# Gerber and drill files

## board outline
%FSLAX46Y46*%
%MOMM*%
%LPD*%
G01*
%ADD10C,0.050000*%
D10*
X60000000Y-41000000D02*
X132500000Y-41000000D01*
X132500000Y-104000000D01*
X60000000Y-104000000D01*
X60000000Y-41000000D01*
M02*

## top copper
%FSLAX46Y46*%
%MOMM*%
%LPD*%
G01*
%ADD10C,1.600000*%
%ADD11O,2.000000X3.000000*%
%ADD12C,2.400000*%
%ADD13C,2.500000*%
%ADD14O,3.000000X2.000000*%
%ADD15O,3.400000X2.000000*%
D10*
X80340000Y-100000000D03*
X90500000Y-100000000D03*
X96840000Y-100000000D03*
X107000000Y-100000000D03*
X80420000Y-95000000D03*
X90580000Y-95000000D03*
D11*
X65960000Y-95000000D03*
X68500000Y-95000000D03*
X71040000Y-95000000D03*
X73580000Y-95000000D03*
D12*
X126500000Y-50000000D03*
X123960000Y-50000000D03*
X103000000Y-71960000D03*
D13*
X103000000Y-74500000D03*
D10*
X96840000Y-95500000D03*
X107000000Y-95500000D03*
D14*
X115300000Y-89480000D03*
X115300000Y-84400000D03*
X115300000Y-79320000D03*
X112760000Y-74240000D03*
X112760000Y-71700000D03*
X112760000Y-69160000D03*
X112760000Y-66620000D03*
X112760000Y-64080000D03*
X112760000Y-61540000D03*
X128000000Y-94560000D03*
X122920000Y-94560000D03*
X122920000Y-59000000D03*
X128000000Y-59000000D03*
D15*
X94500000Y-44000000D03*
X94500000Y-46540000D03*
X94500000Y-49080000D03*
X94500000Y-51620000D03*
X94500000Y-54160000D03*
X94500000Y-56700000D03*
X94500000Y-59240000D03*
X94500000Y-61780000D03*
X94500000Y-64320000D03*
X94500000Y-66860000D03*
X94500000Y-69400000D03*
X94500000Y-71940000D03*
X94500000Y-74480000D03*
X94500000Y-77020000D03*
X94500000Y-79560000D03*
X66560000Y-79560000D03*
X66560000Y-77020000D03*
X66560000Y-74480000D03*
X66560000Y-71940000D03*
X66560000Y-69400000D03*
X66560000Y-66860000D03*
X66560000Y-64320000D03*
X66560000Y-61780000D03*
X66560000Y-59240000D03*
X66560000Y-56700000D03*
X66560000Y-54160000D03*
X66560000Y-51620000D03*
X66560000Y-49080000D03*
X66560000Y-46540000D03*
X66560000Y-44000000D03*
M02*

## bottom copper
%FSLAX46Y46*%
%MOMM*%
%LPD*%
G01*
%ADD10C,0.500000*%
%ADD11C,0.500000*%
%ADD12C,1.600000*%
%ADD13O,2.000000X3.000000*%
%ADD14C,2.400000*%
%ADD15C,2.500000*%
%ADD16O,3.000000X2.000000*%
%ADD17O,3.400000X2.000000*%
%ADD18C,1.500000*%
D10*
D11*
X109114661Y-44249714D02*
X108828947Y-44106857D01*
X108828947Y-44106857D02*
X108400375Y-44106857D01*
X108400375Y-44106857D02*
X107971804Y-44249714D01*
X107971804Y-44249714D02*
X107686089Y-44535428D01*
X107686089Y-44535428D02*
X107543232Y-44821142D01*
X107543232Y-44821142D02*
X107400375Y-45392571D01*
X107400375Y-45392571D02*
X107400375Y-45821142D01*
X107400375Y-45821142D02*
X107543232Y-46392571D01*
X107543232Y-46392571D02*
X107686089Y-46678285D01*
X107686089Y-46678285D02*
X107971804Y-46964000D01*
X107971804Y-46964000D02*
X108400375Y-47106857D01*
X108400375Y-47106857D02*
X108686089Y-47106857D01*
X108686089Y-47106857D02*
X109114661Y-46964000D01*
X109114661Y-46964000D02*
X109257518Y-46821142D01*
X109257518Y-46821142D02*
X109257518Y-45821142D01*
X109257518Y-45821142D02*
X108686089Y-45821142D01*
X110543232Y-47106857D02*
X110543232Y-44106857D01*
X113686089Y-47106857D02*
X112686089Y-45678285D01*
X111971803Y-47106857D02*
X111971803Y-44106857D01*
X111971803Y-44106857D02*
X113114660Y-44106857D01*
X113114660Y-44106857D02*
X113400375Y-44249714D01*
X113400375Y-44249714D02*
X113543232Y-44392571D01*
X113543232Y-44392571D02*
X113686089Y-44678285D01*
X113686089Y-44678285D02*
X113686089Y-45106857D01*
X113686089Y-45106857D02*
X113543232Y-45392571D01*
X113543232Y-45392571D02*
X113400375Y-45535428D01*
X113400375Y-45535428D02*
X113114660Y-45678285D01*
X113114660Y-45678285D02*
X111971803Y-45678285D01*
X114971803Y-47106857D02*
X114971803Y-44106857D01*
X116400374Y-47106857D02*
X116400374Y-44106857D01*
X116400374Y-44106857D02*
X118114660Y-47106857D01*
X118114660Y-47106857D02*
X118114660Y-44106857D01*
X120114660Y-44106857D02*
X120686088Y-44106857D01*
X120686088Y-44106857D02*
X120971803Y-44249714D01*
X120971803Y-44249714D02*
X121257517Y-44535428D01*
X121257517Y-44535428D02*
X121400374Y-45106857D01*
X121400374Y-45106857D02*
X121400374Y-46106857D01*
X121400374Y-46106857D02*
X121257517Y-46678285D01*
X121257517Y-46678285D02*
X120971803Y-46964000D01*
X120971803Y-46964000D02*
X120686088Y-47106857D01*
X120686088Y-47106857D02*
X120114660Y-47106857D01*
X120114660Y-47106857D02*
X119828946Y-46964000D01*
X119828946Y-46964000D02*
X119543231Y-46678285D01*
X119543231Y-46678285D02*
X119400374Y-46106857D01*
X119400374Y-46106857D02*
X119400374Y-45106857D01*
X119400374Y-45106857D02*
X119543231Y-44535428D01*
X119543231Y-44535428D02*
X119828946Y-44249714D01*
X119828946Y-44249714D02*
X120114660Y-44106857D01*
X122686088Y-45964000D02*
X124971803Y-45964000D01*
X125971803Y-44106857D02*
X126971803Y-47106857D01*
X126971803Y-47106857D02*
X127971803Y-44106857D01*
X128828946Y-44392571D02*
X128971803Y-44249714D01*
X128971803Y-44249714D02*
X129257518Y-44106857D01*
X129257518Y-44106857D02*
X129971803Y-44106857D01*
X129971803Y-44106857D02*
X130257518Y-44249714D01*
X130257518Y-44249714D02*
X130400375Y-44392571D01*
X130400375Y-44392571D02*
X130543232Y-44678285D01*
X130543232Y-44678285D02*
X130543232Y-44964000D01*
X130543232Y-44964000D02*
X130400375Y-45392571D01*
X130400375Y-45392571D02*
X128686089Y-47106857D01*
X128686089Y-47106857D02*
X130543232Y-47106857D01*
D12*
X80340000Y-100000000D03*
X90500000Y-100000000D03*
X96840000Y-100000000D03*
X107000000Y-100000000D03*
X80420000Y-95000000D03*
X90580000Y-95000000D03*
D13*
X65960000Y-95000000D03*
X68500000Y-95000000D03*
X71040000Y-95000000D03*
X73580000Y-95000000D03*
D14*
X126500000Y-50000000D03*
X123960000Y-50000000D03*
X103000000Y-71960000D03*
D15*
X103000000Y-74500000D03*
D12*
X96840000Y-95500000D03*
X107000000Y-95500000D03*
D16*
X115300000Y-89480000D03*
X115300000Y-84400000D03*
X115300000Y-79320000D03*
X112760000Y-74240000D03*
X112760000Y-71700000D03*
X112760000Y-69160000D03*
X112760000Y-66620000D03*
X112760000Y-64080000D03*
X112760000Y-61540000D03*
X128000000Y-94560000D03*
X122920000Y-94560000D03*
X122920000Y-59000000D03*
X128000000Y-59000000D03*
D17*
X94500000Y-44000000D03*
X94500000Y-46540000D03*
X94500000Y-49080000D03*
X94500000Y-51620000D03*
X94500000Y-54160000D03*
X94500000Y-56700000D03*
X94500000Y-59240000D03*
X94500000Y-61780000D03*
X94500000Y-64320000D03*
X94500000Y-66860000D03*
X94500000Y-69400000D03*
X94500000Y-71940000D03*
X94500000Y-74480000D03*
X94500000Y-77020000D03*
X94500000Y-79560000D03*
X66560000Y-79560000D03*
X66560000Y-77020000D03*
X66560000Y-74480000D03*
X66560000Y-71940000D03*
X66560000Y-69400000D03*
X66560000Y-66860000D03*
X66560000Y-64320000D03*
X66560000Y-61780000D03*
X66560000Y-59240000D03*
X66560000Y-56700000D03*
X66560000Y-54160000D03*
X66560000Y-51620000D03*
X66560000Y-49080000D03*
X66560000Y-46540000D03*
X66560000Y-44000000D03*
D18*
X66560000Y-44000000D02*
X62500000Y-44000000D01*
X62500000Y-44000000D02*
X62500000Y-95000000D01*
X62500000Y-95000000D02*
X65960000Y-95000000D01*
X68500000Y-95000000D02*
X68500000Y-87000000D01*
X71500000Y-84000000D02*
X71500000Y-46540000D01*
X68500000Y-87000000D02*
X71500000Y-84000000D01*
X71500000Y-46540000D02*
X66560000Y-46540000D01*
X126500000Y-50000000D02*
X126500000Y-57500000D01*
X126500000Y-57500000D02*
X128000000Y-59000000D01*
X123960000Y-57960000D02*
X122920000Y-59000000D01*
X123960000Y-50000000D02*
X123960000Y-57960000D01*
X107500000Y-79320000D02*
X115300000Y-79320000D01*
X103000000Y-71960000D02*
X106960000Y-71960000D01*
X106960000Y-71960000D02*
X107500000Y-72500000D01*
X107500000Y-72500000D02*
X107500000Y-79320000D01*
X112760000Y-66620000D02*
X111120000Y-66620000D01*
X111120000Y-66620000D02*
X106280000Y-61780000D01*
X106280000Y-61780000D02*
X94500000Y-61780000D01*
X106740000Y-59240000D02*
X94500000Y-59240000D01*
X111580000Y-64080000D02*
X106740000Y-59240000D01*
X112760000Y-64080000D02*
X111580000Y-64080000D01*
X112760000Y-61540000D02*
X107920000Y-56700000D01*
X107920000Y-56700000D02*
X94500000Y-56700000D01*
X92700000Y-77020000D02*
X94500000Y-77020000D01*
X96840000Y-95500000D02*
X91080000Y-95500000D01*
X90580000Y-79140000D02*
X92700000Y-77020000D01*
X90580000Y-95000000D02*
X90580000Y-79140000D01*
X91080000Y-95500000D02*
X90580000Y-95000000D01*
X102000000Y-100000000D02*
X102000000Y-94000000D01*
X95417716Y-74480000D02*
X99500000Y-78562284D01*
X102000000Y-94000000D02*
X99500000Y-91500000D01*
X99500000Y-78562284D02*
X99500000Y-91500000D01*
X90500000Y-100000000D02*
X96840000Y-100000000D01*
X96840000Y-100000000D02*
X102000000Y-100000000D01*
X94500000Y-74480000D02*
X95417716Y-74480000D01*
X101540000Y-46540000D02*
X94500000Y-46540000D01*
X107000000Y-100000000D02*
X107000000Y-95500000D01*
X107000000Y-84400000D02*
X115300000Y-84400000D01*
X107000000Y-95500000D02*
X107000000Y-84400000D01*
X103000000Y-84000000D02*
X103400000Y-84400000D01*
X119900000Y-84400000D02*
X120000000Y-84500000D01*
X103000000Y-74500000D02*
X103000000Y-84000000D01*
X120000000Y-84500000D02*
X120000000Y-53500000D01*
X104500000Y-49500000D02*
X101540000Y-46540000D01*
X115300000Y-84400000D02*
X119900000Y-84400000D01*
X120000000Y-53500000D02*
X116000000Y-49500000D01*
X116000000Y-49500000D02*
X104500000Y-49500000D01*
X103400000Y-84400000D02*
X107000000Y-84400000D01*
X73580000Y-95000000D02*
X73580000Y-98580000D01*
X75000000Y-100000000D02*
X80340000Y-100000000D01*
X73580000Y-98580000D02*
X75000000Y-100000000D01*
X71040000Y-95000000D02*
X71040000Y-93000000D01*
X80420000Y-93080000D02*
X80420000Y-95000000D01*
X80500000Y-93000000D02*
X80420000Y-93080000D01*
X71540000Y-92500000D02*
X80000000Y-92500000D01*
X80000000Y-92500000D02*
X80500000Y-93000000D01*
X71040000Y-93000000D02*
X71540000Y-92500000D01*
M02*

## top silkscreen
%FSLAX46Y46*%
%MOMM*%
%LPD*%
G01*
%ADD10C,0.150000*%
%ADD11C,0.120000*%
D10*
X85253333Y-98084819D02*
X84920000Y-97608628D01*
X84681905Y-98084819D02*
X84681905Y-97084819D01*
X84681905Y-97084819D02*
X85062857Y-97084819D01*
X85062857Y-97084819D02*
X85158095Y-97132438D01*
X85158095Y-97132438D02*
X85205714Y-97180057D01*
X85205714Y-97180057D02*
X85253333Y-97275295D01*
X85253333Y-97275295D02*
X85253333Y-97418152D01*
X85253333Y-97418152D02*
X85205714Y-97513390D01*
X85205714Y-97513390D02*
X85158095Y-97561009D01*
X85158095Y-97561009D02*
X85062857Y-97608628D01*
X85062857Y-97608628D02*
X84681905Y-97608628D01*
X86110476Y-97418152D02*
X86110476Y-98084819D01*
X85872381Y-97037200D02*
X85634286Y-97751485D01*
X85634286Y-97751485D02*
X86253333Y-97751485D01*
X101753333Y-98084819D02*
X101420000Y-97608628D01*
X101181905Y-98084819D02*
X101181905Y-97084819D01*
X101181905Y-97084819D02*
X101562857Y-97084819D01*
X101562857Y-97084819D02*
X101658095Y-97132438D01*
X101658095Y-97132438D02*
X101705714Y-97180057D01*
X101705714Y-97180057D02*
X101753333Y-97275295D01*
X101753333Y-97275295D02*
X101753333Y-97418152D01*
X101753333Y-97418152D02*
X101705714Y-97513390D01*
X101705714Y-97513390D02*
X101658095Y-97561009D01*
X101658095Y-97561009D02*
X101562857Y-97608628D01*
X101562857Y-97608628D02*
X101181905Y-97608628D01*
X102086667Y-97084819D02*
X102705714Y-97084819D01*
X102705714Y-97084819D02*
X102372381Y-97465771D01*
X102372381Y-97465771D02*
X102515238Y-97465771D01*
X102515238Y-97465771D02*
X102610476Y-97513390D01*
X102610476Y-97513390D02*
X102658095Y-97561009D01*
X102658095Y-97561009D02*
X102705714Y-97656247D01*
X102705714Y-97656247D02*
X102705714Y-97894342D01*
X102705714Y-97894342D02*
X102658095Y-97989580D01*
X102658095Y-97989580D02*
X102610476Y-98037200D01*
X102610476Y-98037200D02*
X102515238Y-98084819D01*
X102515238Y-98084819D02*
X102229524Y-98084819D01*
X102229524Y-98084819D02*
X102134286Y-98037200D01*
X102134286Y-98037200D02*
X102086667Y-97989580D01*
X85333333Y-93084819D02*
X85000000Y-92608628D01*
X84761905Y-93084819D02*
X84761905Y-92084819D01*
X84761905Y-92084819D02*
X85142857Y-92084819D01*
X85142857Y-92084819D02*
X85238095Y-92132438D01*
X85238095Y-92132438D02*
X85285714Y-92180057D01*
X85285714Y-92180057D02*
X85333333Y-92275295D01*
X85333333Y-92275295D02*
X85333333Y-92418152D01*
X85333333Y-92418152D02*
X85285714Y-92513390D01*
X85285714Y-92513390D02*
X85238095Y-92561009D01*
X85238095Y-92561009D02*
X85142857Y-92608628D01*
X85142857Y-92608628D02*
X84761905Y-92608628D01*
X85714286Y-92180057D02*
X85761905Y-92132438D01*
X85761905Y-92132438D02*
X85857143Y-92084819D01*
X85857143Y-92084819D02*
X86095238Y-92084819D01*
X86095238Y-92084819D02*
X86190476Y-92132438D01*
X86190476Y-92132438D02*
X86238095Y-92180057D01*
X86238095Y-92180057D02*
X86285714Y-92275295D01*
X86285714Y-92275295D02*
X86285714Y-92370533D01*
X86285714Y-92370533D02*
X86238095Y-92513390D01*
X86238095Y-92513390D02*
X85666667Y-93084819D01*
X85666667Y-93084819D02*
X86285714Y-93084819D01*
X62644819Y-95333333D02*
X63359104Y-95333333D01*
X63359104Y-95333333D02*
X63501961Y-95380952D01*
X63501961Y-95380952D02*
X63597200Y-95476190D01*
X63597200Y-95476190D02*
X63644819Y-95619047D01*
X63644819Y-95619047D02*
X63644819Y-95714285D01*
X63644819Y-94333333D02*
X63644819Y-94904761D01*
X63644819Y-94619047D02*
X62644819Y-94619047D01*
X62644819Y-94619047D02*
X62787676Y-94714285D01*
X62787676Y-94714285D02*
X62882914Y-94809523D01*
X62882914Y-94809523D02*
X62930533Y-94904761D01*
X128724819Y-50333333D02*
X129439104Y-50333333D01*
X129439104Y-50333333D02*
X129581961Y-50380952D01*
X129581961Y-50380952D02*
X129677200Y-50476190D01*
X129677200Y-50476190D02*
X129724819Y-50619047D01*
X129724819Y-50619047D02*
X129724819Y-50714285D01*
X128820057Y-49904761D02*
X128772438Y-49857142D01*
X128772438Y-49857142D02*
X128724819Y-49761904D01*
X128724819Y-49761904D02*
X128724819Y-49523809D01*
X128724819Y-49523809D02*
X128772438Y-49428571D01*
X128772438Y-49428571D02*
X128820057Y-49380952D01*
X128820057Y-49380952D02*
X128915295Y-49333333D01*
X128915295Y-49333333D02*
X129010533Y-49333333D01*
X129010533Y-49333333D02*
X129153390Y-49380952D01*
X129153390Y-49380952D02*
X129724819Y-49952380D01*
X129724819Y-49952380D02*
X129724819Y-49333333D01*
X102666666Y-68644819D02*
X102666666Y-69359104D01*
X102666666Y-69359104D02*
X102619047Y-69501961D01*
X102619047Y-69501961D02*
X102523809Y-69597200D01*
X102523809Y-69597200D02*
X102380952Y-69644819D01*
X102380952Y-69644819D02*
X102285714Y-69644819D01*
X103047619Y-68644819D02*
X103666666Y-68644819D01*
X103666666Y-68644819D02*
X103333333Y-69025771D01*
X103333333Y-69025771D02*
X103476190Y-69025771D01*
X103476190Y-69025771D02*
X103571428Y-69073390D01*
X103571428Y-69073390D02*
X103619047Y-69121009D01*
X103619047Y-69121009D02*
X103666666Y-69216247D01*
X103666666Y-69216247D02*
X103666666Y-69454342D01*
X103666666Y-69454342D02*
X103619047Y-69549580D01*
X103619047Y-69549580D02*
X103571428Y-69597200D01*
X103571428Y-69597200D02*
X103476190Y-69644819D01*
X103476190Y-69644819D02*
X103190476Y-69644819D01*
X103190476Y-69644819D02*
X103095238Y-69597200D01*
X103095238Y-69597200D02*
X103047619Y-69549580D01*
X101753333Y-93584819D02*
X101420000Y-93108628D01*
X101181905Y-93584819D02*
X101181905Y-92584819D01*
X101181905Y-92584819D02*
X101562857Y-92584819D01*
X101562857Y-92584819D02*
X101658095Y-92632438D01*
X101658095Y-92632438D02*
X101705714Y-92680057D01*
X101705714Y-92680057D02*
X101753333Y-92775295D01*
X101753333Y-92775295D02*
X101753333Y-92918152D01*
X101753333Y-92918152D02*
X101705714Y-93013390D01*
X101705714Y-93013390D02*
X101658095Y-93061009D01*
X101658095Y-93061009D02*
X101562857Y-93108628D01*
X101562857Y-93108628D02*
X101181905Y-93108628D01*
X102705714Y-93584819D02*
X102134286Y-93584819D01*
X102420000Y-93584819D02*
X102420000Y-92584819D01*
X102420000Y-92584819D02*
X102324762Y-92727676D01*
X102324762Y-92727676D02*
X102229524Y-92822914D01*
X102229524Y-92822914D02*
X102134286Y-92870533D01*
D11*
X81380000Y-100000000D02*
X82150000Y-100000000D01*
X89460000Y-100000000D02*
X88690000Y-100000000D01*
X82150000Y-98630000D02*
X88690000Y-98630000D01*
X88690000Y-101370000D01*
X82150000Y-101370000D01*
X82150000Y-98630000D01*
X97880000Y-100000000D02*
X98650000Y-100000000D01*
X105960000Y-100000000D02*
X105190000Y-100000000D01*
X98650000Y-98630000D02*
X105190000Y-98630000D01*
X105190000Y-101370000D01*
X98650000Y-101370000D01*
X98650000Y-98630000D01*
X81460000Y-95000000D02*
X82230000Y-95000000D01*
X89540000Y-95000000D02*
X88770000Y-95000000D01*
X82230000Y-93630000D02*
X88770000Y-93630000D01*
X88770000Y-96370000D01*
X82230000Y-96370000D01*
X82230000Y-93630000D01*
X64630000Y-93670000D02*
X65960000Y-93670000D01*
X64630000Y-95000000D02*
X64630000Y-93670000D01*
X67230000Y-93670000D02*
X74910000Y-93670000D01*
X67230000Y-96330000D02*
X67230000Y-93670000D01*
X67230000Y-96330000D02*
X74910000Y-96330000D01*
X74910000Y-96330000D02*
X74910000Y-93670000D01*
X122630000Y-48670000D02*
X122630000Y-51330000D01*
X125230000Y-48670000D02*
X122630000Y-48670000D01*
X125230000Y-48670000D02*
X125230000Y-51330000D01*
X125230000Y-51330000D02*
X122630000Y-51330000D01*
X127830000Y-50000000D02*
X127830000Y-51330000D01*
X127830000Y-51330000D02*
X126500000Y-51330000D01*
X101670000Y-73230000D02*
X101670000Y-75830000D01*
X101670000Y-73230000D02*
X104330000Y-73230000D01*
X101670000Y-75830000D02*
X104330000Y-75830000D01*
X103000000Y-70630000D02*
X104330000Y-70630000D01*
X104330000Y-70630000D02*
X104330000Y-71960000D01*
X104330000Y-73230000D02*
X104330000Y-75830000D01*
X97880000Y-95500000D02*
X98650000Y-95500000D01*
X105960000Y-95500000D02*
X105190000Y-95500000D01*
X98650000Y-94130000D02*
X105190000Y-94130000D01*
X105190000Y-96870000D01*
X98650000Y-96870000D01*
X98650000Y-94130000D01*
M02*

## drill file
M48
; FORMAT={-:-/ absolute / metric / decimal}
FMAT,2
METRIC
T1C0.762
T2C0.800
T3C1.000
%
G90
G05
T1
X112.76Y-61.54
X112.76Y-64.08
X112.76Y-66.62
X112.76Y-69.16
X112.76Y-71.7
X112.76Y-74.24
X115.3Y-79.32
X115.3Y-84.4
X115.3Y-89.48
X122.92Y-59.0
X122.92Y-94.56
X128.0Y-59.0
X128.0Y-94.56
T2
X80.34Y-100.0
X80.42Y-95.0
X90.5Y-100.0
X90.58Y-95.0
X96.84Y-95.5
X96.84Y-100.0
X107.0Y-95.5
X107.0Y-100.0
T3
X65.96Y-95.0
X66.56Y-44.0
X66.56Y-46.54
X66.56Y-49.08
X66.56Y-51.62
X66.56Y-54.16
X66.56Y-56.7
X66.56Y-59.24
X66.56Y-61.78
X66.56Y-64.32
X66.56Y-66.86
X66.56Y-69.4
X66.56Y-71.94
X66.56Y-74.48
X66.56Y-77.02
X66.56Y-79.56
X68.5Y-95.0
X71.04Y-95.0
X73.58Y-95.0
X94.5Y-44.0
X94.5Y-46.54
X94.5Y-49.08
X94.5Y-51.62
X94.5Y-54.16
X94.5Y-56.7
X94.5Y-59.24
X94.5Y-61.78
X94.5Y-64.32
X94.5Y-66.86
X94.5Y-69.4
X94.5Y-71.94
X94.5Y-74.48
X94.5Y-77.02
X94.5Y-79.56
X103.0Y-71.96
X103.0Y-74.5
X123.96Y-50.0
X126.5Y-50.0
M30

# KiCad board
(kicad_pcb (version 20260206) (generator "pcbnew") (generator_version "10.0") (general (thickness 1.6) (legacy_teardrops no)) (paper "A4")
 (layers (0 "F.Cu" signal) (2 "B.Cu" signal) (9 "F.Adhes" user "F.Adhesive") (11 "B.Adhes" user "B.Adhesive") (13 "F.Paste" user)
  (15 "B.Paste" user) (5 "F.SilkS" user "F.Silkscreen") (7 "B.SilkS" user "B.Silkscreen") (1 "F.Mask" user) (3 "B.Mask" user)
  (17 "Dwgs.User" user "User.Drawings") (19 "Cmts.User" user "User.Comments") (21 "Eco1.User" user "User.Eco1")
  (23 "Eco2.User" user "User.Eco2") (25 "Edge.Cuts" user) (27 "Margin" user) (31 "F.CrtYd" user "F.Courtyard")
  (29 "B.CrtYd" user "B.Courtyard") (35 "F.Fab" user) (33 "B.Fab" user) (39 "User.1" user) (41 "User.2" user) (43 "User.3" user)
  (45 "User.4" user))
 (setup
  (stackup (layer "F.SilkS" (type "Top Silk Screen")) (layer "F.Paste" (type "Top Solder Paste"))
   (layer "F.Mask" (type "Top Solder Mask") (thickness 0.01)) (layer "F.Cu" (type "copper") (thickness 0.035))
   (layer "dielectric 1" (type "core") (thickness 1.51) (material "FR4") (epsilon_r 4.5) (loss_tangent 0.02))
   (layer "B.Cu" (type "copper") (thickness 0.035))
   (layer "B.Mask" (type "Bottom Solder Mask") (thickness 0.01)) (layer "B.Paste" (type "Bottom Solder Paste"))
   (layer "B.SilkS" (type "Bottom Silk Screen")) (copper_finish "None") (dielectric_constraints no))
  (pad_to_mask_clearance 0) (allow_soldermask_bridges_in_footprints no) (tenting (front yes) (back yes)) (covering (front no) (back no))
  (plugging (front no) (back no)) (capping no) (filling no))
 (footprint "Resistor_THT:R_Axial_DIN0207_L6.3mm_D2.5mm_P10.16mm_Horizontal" (layer "F.Cu") (at 80.34 100)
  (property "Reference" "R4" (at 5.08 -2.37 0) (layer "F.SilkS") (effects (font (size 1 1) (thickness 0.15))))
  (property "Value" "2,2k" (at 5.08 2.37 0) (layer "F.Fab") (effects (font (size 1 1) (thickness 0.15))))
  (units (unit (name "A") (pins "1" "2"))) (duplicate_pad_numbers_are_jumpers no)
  (fp_line (start 1.04 0) (end 1.81 0) (stroke (width 0.12) (type solid)) (layer "F.SilkS"))
  (fp_line (start 9.12 0) (end 8.35 0) (stroke (width 0.12) (type solid)) (layer "F.SilkS"))
  (fp_rect (start 1.81 -1.37) (end 8.35 1.37) (stroke (width 0.12) (type solid)) (fill no) (layer "F.SilkS"))
  (pad "1" thru_hole circle (at 0 0) (size 1.6 1.6) (drill 0.8) (layers "*.Cu" "*.Mask") (remove_unused_layers no) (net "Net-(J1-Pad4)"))
  (pad "2" thru_hole circle (at 10.16 0) (size 1.6 1.6) (drill 0.8) (layers "*.Cu" "*.Mask") (remove_unused_layers no)
   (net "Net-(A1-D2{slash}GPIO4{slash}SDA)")))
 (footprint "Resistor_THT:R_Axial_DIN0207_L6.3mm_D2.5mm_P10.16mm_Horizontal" (layer "F.Cu") (at 96.84 100)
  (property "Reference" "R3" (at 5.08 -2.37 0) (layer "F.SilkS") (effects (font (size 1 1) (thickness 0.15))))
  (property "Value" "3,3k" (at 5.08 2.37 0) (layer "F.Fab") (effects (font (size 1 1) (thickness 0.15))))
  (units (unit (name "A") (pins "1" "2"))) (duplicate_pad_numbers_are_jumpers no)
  (fp_line (start 1.04 0) (end 1.81 0) (stroke (width 0.12) (type solid)) (layer "F.SilkS"))
  (fp_line (start 9.12 0) (end 8.35 0) (stroke (width 0.12) (type solid)) (layer "F.SilkS"))
  (fp_rect (start 1.81 -1.37) (end 8.35 1.37) (stroke (width 0.12) (type solid)) (fill no) (layer "F.SilkS"))
  (pad "1" thru_hole circle (at 0 0) (size 1.6 1.6) (drill 0.8) (layers "*.Cu" "*.Mask") (remove_unused_layers no)
   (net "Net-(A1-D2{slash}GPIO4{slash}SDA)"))
  (pad "2" thru_hole circle (at 10.16 0) (size 1.6 1.6) (drill 0.8) (layers "*.Cu" "*.Mask") (remove_unused_layers no) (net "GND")))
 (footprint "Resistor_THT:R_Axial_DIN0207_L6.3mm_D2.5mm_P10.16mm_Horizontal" (layer "F.Cu") (at 80.42 95)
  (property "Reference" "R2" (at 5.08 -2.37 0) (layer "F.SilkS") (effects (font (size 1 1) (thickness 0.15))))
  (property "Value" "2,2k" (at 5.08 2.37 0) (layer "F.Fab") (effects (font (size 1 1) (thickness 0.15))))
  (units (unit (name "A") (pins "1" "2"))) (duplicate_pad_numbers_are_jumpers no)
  (fp_line (start 1.04 0) (end 1.81 0) (stroke (width 0.12) (type solid)) (layer "F.SilkS"))
  (fp_line (start 9.12 0) (end 8.35 0) (stroke (width 0.12) (type solid)) (layer "F.SilkS"))
  (fp_rect (start 1.81 -1.37) (end 8.35 1.37) (stroke (width 0.12) (type solid)) (fill no) (layer "F.SilkS"))
  (pad "1" thru_hole circle (at 0 0) (size 1.6 1.6) (drill 0.8) (layers "*.Cu" "*.Mask") (remove_unused_layers no) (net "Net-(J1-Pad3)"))
  (pad "2" thru_hole circle (at 10.16 0) (size 1.6 1.6) (drill 0.8) (layers "*.Cu" "*.Mask") (remove_unused_layers no)
   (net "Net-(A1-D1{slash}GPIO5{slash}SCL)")))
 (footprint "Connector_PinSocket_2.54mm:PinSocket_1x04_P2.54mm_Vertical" (layer "F.Cu") (at 65.96 95 90)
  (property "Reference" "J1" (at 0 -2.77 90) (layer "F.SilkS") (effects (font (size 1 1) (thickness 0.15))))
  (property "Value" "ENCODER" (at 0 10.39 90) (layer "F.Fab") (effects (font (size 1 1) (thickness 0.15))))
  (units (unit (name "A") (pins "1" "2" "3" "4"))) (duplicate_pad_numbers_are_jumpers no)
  (fp_line (start 1.33 -1.33) (end 1.33 0) (stroke (width 0.12) (type solid)) (layer "F.SilkS"))
  (fp_line (start 0 -1.33) (end 1.33 -1.33) (stroke (width 0.12) (type solid)) (layer "F.SilkS"))
  (fp_line (start 1.33 1.27) (end 1.33 8.95) (stroke (width 0.12) (type solid)) (layer "F.SilkS"))
  (fp_line (start -1.33 1.27) (end 1.33 1.27) (stroke (width 0.12) (type solid)) (layer "F.SilkS"))
  (fp_line (start -1.33 1.27) (end -1.33 8.95) (stroke (width 0.12) (type solid)) (layer "F.SilkS"))
  (fp_line (start -1.33 8.95) (end 1.33 8.95) (stroke (width 0.12) (type solid)) (layer "F.SilkS"))
  (pad "1" thru_hole oval (at 0 0 90) (size 3 2) (drill 1) (layers "*.Cu" "*.Mask") (remove_unused_layers no) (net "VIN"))
  (pad "2" thru_hole oval (at 0 2.54 90) (size 3 2) (drill 1) (layers "*.Cu" "*.Mask") (remove_unused_layers no) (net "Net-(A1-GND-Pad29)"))
  (pad "3" thru_hole oval (at 0 5.08 90) (size 3 2) (drill 1) (layers "*.Cu" "*.Mask") (remove_unused_layers no) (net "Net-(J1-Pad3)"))
  (pad "4" thru_hole oval (at 0 7.62 90) (size 3 2) (drill 1) (layers "*.Cu" "*.Mask") (remove_unused_layers no) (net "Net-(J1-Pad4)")))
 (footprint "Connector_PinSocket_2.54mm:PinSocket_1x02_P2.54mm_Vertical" (layer "F.Cu") (at 126.5 50 -90)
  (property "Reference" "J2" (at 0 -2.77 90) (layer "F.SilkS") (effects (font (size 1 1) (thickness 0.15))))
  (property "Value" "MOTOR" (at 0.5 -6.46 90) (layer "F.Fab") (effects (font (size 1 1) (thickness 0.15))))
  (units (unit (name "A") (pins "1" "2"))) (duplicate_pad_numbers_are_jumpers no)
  (fp_line (start -1.33 3.87) (end 1.33 3.87) (stroke (width 0.12) (type solid)) (layer "F.SilkS"))
  (fp_line (start -1.33 1.27) (end -1.33 3.87) (stroke (width 0.12) (type solid)) (layer "F.SilkS"))
  (fp_line (start -1.33 1.27) (end 1.33 1.27) (stroke (width 0.12) (type solid)) (layer "F.SilkS"))
  (fp_line (start 1.33 1.27) (end 1.33 3.87) (stroke (width 0.12) (type solid)) (layer "F.SilkS"))
  (fp_line (start 0 -1.33) (end 1.33 -1.33) (stroke (width 0.12) (type solid)) (layer "F.SilkS"))
  (fp_line (start 1.33 -1.33) (end 1.33 0) (stroke (width 0.12) (type solid)) (layer "F.SilkS"))
  (pad "1" thru_hole circle (at 0 0 270) (size 2.4 2.4) (drill 1) (layers "*.Cu" "*.Mask") (remove_unused_layers no) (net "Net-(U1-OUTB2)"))
  (pad "2" thru_hole circle (at 0 2.54 270) (size 2.4 2.4) (drill 1) (layers "*.Cu" "*.Mask") (remove_unused_layers no)
   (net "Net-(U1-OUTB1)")))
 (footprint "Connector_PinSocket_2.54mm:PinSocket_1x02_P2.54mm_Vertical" (layer "F.Cu") (at 103 71.96)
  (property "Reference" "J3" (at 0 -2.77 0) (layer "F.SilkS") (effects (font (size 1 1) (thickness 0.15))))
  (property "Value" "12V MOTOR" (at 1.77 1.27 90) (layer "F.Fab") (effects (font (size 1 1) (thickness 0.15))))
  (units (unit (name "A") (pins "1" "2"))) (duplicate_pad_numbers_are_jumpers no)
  (fp_line (start -1.33 1.27) (end -1.33 3.87) (stroke (width 0.12) (type solid)) (layer "F.SilkS"))
  (fp_line (start -1.33 1.27) (end 1.33 1.27) (stroke (width 0.12) (type solid)) (layer "F.SilkS"))
  (fp_line (start -1.33 3.87) (end 1.33 3.87) (stroke (width 0.12) (type solid)) (layer "F.SilkS"))
  (fp_line (start 0 -1.33) (end 1.33 -1.33) (stroke (width 0.12) (type solid)) (layer "F.SilkS"))
  (fp_line (start 1.33 -1.33) (end 1.33 0) (stroke (width 0.12) (type solid)) (layer "F.SilkS"))
  (fp_line (start 1.33 1.27) (end 1.33 3.87) (stroke (width 0.12) (type solid)) (layer "F.SilkS"))
  (pad "1" thru_hole circle (at 0 0) (size 2.4 2.4) (drill 1) (layers "*.Cu" "*.Mask") (remove_unused_layers no) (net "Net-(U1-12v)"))
  (pad "2" thru_hole circle (at 0 2.54) (size 2.5 2.5) (drill 1) (layers "*.Cu" "*.Mask") (remove_unused_layers no) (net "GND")))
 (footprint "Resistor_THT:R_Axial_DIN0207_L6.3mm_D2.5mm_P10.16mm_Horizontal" (layer "F.Cu") (at 96.84 95.5)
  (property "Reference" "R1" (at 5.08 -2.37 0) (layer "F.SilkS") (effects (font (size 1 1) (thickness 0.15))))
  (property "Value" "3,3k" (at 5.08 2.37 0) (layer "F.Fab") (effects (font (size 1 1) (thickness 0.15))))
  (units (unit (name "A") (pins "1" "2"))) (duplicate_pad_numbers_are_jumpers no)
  (fp_line (start 1.04 0) (end 1.81 0) (stroke (width 0.12) (type solid)) (layer "F.SilkS"))
  (fp_line (start 9.12 0) (end 8.35 0) (stroke (width 0.12) (type solid)) (layer "F.SilkS"))
  (fp_rect (start 1.81 -1.37) (end 8.35 1.37) (stroke (width 0.12) (type solid)) (fill no) (layer "F.SilkS"))
  (pad "1" thru_hole circle (at 0 0) (size 1.6 1.6) (drill 0.8) (layers "*.Cu" "*.Mask") (remove_unused_layers no)
   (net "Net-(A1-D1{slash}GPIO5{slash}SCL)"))
  (pad "2" thru_hole circle (at 10.16 0) (size 1.6 1.6) (drill 0.8) (layers "*.Cu" "*.Mask") (remove_unused_layers no) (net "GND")))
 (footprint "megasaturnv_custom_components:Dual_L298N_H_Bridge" (layer "B.Cu") (at 110.22 97.1 90)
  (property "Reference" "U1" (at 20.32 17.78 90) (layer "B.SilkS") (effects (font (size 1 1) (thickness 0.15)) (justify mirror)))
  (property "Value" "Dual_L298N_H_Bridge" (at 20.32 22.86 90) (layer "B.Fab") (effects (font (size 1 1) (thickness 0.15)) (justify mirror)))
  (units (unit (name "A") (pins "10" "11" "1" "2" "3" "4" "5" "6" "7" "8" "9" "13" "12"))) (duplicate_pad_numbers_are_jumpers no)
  (pad "1" thru_hole oval (at 7.62 5.08 90) (size 2 3) (drill 0.762) (layers "*.Cu" "*.Mask") (remove_unused_layers no)
   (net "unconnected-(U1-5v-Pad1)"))
  (pad "2" thru_hole oval (at 12.7 5.08 90) (size 2 3) (drill 0.762) (layers "*.Cu" "*.Mask") (remove_unused_layers no) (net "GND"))
  (pad "3" thru_hole oval (at 17.78 5.08 90) (size 2 3) (drill 0.762) (layers "*.Cu" "*.Mask") (remove_unused_layers no)
   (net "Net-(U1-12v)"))
  (pad "4" thru_hole oval (at 22.86 2.54 90) (size 2 3) (drill 0.762) (layers "*.Cu" "*.Mask") (remove_unused_layers no)
   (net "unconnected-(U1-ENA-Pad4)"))
  (pad "5" thru_hole oval (at 25.4 2.54 90) (size 2 3) (drill 0.762) (layers "*.Cu" "*.Mask") (remove_unused_layers no)
   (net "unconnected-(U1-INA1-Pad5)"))
  (pad "6" thru_hole oval (at 27.94 2.54 90) (size 2 3) (drill 0.762) (layers "*.Cu" "*.Mask") (remove_unused_layers no)
   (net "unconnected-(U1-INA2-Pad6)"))
  (pad "7" thru_hole oval (at 30.48 2.54 90) (size 2 3) (drill 0.762) (layers "*.Cu" "*.Mask") (remove_unused_layers no)
   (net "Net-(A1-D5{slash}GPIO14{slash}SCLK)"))
  (pad "8" thru_hole oval (at 33.02 2.54 90) (size 2 3) (drill 0.762) (layers "*.Cu" "*.Mask") (remove_unused_layers no)
   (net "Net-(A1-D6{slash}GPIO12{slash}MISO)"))
  (pad "9" thru_hole oval (at 35.56 2.54 90) (size 2 3) (drill 0.762) (layers "*.Cu" "*.Mask") (remove_unused_layers no)
   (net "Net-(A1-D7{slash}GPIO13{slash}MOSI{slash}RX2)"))
  (pad "10" thru_hole oval (at 2.54 17.78 90) (size 2 3) (drill 0.762) (layers "*.Cu" "*.Mask") (remove_unused_layers no)
   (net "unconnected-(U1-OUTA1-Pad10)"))
  (pad "11" thru_hole oval (at 2.54 12.7 90) (size 2 3) (drill 0.762) (layers "*.Cu" "*.Mask") (remove_unused_layers no)
   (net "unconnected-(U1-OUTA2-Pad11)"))
  (pad "12" thru_hole oval (at 38.1 12.7 90) (size 2 3) (drill 0.762) (layers "*.Cu" "*.Mask") (remove_unused_layers no)
   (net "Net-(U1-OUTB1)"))
  (pad "13" thru_hole oval (at 38.1 17.78 90) (size 2 3) (drill 0.762) (layers "*.Cu" "*.Mask") (remove_unused_layers no)
   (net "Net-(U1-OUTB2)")))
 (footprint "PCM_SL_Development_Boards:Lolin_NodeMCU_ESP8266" (layer "B.Cu") (at 80.53 61.78 180)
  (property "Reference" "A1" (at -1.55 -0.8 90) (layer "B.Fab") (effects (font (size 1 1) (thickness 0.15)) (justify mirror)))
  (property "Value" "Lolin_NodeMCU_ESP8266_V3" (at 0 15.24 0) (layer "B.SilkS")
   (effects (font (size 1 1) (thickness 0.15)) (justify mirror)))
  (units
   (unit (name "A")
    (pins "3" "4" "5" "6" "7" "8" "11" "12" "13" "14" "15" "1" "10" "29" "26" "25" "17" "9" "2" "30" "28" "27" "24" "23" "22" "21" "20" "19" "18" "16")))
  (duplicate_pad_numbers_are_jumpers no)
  (pad "1" thru_hole oval (at -13.97 17.78 270) (size 2 3.4) (drill 1) (layers "*.Cu" "*.Mask") (remove_unused_layers no)
   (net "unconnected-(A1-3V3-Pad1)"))
  (pad "2" thru_hole oval (at -13.97 15.24 270) (size 2 3.4) (drill 1) (layers "*.Cu" "*.Mask") (remove_unused_layers no) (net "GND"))
  (pad "3" thru_hole oval (at -13.97 12.7 270) (size 2 3.4) (drill 1) (layers "*.Cu" "*.Mask") (remove_unused_layers no)
   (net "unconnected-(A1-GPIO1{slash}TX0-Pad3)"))
  (pad "4" thru_hole oval (at -13.97 10.16 270) (size 2 3.4) (drill 1) (layers "*.Cu" "*.Mask") (remove_unused_layers no)
   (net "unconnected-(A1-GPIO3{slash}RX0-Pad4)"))
  (pad "5" thru_hole oval (at -13.97 7.62 270) (size 2 3.4) (drill 1) (layers "*.Cu" "*.Mask") (remove_unused_layers no)
   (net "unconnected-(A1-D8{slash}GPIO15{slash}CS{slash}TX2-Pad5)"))
  (pad "6" thru_hole oval (at -13.97 5.08 270) (size 2 3.4) (drill 1) (layers "*.Cu" "*.Mask") (remove_unused_layers no)
   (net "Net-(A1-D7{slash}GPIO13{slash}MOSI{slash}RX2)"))
  (pad "7" thru_hole oval (at -13.97 2.54 270) (size 2 3.4) (drill 1) (layers "*.Cu" "*.Mask") (remove_unused_layers no)
   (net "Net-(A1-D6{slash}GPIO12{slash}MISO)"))
  (pad "8" thru_hole oval (at -13.97 0 270) (size 2 3.4) (drill 1) (layers "*.Cu" "*.Mask") (remove_unused_layers no)
   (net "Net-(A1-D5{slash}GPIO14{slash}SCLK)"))
  (pad "9" thru_hole oval (at -13.97 -2.54 270) (size 2 3.4) (drill 1) (layers "*.Cu" "*.Mask") (remove_unused_layers no)
   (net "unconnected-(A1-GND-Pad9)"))
  (pad "10" thru_hole oval (at -13.97 -5.08 270) (size 2 3.4) (drill 1) (layers "*.Cu" "*.Mask") (remove_unused_layers no)
   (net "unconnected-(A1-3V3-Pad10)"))
  (pad "11" thru_hole oval (at -13.97 -7.62 270) (size 2 3.4) (drill 1) (layers "*.Cu" "*.Mask") (remove_unused_layers no)
   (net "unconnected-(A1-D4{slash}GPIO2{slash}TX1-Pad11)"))
  (pad "12" thru_hole oval (at -13.97 -10.16 270) (size 2 3.4) (drill 1) (layers "*.Cu" "*.Mask") (remove_unused_layers no)
   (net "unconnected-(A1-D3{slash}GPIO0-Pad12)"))
  (pad "13" thru_hole oval (at -13.97 -12.7 270) (size 2 3.4) (drill 1) (layers "*.Cu" "*.Mask") (remove_unused_layers no)
   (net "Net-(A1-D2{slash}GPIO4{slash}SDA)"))
  (pad "14" thru_hole oval (at -13.97 -15.24 270) (size 2 3.4) (drill 1) (layers "*.Cu" "*.Mask") (remove_unused_layers no)
   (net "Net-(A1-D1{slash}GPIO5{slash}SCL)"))
  (pad "15" thru_hole oval (at -13.97 -17.78 270) (size 2 3.4) (drill 1) (layers "*.Cu" "*.Mask") (remove_unused_layers no)
   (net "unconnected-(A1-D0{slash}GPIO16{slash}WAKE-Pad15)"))
  (pad "16" thru_hole oval (at 13.97 -17.78 270) (size 2 3.4) (drill 1) (layers "*.Cu" "*.Mask") (remove_unused_layers no)
   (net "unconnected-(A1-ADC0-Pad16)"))
  (pad "17" thru_hole oval (at 13.97 -15.24 270) (size 2 3.4) (drill 1) (layers "*.Cu" "*.Mask") (remove_unused_layers no)
   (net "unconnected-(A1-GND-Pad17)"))
  (pad "18" thru_hole oval (at 13.97 -12.7 270) (size 2 3.4) (drill 1) (layers "*.Cu" "*.Mask") (remove_unused_layers no)
   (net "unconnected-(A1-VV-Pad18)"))
  (pad "19" thru_hole oval (at 13.97 -10.16 270) (size 2 3.4) (drill 1) (layers "*.Cu" "*.Mask") (remove_unused_layers no)
   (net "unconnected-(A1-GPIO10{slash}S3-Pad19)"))
  (pad "20" thru_hole oval (at 13.97 -7.62 270) (size 2 3.4) (drill 1) (layers "*.Cu" "*.Mask") (remove_unused_layers no)
   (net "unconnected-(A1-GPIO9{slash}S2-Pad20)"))
  (pad "21" thru_hole oval (at 13.97 -5.08 270) (size 2 3.4) (drill 1) (layers "*.Cu" "*.Mask") (remove_unused_layers no)
   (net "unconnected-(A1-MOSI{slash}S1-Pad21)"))
  (pad "22" thru_hole oval (at 13.97 -2.54 270) (size 2 3.4) (drill 1) (layers "*.Cu" "*.Mask") (remove_unused_layers no)
   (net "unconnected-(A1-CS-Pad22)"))
  (pad "23" thru_hole oval (at 13.97 0 270) (size 2 3.4) (drill 1) (layers "*.Cu" "*.Mask") (remove_unused_layers no)
   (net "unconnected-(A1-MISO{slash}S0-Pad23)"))
  (pad "24" thru_hole oval (at 13.97 2.54 270) (size 2 3.4) (drill 1) (layers "*.Cu" "*.Mask") (remove_unused_layers no)
   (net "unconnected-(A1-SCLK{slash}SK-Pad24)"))
  (pad "25" thru_hole oval (at 13.97 5.08 270) (size 2 3.4) (drill 1) (layers "*.Cu" "*.Mask") (remove_unused_layers no)
   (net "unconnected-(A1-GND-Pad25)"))
  (pad "26" thru_hole oval (at 13.97 7.62 270) (size 2 3.4) (drill 1) (layers "*.Cu" "*.Mask") (remove_unused_layers no) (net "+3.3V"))
  (pad "27" thru_hole oval (at 13.97 10.16 270) (size 2 3.4) (drill 1) (layers "*.Cu" "*.Mask") (remove_unused_layers no)
   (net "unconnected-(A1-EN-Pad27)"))
  (pad "28" thru_hole oval (at 13.97 12.7 270) (size 2 3.4) (drill 1) (layers "*.Cu" "*.Mask") (remove_unused_layers no)
   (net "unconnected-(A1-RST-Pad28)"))
  (pad "29" thru_hole oval (at 13.97 15.24 270) (size 2 3.4) (drill 1) (layers "*.Cu" "*.Mask") (remove_unused_layers no)
   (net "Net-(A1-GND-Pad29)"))
  (pad "30" thru_hole oval (at 13.97 17.78 270) (size 2 3.4) (drill 1) (layers "*.Cu" "*.Mask") (remove_unused_layers no) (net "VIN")))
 (gr_rect (start 60 41) (end 132.5 104) (stroke (width 0.05) (type default)) (fill no) (layer "Edge.Cuts"))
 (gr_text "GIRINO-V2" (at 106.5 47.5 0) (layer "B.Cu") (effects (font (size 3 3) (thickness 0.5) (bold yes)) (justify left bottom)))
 (segment (start 66.56 44) (end 62.5 44) (width 1.5) (layer "B.Cu") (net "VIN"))
 (segment (start 62.5 44) (end 62.5 95) (width 1.5) (layer "B.Cu") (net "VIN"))
 (segment (start 62.5 95) (end 65.96 95) (width 1.5) (layer "B.Cu") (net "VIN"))
 (segment (start 68.5 95) (end 68.5 87) (width 1.5) (layer "B.Cu") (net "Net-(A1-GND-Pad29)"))
 (segment (start 71.5 84) (end 71.5 46.54) (width 1.5) (layer "B.Cu") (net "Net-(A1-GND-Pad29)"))
 (segment (start 68.5 87) (end 71.5 84) (width 1.5) (layer "B.Cu") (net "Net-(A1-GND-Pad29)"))
 (segment (start 71.5 46.54) (end 66.56 46.54) (width 1.5) (layer "B.Cu") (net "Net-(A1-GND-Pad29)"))
 (segment (start 126.5 50) (end 126.5 57.5) (width 1.5) (layer "B.Cu") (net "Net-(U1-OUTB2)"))
 (segment (start 126.5 57.5) (end 128 59) (width 1.5) (layer "B.Cu") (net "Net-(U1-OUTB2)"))
 (segment (start 123.96 57.96) (end 122.92 59) (width 1.5) (layer "B.Cu") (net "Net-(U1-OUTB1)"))
 (segment (start 123.96 50) (end 123.96 57.96) (width 1.5) (layer "B.Cu") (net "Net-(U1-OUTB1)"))
 (segment (start 107.5 79.32) (end 115.3 79.32) (width 1.5) (layer "B.Cu") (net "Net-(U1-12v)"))
 (segment (start 103 71.96) (end 106.96 71.96) (width 1.5) (layer "B.Cu") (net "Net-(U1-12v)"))
 (segment (start 106.96 71.96) (end 107.5 72.5) (width 1.5) (layer "B.Cu") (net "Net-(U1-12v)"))
 (segment (start 107.5 72.5) (end 107.5 79.32) (width 1.5) (layer "B.Cu") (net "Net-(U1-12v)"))
 (segment (start 112.76 66.62) (end 111.12 66.62) (width 1.5) (layer "B.Cu") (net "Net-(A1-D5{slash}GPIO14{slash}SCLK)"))
 (segment (start 111.12 66.62) (end 106.28 61.78) (width 1.5) (layer "B.Cu") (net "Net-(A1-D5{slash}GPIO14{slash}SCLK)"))
 (segment (start 106.28 61.78) (end 94.5 61.78) (width 1.5) (layer "B.Cu") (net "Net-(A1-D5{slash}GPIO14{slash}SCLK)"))
 (segment (start 106.74 59.24) (end 94.5 59.24) (width 1.5) (layer "B.Cu") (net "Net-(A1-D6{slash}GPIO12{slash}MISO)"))
 (segment (start 111.58 64.08) (end 106.74 59.24) (width 1.5) (layer "B.Cu") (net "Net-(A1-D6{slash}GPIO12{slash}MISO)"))
 (segment (start 112.76 64.08) (end 111.58 64.08) (width 1.5) (layer "B.Cu") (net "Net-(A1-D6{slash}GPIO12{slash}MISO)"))
 (segment (start 112.76 61.54) (end 107.92 56.7) (width 1.5) (layer "B.Cu") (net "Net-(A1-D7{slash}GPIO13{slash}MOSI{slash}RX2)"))
 (segment (start 107.92 56.7) (end 94.5 56.7) (width 1.5) (layer "B.Cu") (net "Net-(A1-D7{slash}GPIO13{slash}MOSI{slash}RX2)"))
 (segment (start 92.7 77.02) (end 94.5 77.02) (width 1.5) (layer "B.Cu") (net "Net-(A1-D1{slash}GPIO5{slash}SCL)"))
 (segment (start 96.84 95.5) (end 91.08 95.5) (width 1.5) (layer "B.Cu") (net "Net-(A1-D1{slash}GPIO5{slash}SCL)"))
 (segment (start 90.58 79.14) (end 92.7 77.02) (width 1.5) (layer "B.Cu") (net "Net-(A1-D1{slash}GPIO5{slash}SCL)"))
 (segment (start 90.58 95) (end 90.58 79.14) (width 1.5) (layer "B.Cu") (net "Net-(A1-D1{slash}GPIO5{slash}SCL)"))
 (segment (start 91.08 95.5) (end 90.58 95) (width 1.5) (layer "B.Cu") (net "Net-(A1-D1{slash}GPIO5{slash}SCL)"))
 (segment (start 102 100) (end 102 94) (width 1.5) (layer "B.Cu") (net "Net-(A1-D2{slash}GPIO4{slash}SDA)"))
 (segment (start 95.417716 74.48) (end 99.5 78.562284) (width 1.5) (layer "B.Cu") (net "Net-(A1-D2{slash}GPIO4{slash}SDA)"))
 (segment (start 102 94) (end 99.5 91.5) (width 1.5) (layer "B.Cu") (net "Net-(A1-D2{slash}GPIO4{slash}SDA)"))
 (segment (start 99.5 78.562284) (end 99.5 91.5) (width 1.5) (layer "B.Cu") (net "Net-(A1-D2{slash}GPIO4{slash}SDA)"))
 (segment (start 90.5 100) (end 96.84 100) (width 1.5) (layer "B.Cu") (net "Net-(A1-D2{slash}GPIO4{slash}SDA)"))
 (segment (start 96.84 100) (end 102 100) (width 1.5) (layer "B.Cu") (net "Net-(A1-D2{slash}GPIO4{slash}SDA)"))
 (segment (start 94.5 74.48) (end 95.417716 74.48) (width 1.5) (layer "B.Cu") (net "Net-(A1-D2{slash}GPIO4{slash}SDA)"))
 (segment (start 101.54 46.54) (end 94.5 46.54) (width 1.5) (layer "B.Cu") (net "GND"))
 (segment (start 107 100) (end 107 95.5) (width 1.5) (layer "B.Cu") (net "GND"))
 (segment (start 107 84.4) (end 115.3 84.4) (width 1.5) (layer "B.Cu") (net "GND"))
 (segment (start 107 95.5) (end 107 84.4) (width 1.5) (layer "B.Cu") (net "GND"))
 (segment (start 103 84) (end 103.4 84.4) (width 1.5) (layer "B.Cu") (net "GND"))
 (segment (start 119.9 84.4) (end 120 84.5) (width 1.5) (layer "B.Cu") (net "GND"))
 (segment (start 103 74.5) (end 103 84) (width 1.5) (layer "B.Cu") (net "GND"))
 (segment (start 120 84.5) (end 120 53.5) (width 1.5) (layer "B.Cu") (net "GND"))
 (segment (start 104.5 49.5) (end 101.54 46.54) (width 1.5) (layer "B.Cu") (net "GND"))
 (segment (start 115.3 84.4) (end 119.9 84.4) (width 1.5) (layer "B.Cu") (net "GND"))
 (segment (start 120 53.5) (end 116 49.5) (width 1.5) (layer "B.Cu") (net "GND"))
 (segment (start 116 49.5) (end 104.5 49.5) (width 1.5) (layer "B.Cu") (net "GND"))
 (segment (start 103.4 84.4) (end 107 84.4) (width 1.5) (layer "B.Cu") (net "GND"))
 (segment (start 73.58 95) (end 73.58 98.58) (width 1.5) (layer "B.Cu") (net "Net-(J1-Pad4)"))
 (segment (start 75 100) (end 80.34 100) (width 1.5) (layer "B.Cu") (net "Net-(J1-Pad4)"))
 (segment (start 73.58 98.58) (end 75 100) (width 1.5) (layer "B.Cu") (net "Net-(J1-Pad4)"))
 (segment (start 71.04 95) (end 71.04 93) (width 1.5) (layer "B.Cu") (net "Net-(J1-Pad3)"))
 (segment (start 80.42 93.08) (end 80.42 95) (width 1.5) (layer "B.Cu") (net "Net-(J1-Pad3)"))
 (segment (start 80.5 93) (end 80.42 93.08) (width 1.5) (layer "B.Cu") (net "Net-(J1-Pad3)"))
 (segment (start 71.54 92.5) (end 80 92.5) (width 1.5) (layer "B.Cu") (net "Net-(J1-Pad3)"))
 (segment (start 80 92.5) (end 80.5 93) (width 1.5) (layer "B.Cu") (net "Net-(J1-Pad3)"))
 (segment (start 71.04 93) (end 71.54 92.5) (width 1.5) (layer "B.Cu") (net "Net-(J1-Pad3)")))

